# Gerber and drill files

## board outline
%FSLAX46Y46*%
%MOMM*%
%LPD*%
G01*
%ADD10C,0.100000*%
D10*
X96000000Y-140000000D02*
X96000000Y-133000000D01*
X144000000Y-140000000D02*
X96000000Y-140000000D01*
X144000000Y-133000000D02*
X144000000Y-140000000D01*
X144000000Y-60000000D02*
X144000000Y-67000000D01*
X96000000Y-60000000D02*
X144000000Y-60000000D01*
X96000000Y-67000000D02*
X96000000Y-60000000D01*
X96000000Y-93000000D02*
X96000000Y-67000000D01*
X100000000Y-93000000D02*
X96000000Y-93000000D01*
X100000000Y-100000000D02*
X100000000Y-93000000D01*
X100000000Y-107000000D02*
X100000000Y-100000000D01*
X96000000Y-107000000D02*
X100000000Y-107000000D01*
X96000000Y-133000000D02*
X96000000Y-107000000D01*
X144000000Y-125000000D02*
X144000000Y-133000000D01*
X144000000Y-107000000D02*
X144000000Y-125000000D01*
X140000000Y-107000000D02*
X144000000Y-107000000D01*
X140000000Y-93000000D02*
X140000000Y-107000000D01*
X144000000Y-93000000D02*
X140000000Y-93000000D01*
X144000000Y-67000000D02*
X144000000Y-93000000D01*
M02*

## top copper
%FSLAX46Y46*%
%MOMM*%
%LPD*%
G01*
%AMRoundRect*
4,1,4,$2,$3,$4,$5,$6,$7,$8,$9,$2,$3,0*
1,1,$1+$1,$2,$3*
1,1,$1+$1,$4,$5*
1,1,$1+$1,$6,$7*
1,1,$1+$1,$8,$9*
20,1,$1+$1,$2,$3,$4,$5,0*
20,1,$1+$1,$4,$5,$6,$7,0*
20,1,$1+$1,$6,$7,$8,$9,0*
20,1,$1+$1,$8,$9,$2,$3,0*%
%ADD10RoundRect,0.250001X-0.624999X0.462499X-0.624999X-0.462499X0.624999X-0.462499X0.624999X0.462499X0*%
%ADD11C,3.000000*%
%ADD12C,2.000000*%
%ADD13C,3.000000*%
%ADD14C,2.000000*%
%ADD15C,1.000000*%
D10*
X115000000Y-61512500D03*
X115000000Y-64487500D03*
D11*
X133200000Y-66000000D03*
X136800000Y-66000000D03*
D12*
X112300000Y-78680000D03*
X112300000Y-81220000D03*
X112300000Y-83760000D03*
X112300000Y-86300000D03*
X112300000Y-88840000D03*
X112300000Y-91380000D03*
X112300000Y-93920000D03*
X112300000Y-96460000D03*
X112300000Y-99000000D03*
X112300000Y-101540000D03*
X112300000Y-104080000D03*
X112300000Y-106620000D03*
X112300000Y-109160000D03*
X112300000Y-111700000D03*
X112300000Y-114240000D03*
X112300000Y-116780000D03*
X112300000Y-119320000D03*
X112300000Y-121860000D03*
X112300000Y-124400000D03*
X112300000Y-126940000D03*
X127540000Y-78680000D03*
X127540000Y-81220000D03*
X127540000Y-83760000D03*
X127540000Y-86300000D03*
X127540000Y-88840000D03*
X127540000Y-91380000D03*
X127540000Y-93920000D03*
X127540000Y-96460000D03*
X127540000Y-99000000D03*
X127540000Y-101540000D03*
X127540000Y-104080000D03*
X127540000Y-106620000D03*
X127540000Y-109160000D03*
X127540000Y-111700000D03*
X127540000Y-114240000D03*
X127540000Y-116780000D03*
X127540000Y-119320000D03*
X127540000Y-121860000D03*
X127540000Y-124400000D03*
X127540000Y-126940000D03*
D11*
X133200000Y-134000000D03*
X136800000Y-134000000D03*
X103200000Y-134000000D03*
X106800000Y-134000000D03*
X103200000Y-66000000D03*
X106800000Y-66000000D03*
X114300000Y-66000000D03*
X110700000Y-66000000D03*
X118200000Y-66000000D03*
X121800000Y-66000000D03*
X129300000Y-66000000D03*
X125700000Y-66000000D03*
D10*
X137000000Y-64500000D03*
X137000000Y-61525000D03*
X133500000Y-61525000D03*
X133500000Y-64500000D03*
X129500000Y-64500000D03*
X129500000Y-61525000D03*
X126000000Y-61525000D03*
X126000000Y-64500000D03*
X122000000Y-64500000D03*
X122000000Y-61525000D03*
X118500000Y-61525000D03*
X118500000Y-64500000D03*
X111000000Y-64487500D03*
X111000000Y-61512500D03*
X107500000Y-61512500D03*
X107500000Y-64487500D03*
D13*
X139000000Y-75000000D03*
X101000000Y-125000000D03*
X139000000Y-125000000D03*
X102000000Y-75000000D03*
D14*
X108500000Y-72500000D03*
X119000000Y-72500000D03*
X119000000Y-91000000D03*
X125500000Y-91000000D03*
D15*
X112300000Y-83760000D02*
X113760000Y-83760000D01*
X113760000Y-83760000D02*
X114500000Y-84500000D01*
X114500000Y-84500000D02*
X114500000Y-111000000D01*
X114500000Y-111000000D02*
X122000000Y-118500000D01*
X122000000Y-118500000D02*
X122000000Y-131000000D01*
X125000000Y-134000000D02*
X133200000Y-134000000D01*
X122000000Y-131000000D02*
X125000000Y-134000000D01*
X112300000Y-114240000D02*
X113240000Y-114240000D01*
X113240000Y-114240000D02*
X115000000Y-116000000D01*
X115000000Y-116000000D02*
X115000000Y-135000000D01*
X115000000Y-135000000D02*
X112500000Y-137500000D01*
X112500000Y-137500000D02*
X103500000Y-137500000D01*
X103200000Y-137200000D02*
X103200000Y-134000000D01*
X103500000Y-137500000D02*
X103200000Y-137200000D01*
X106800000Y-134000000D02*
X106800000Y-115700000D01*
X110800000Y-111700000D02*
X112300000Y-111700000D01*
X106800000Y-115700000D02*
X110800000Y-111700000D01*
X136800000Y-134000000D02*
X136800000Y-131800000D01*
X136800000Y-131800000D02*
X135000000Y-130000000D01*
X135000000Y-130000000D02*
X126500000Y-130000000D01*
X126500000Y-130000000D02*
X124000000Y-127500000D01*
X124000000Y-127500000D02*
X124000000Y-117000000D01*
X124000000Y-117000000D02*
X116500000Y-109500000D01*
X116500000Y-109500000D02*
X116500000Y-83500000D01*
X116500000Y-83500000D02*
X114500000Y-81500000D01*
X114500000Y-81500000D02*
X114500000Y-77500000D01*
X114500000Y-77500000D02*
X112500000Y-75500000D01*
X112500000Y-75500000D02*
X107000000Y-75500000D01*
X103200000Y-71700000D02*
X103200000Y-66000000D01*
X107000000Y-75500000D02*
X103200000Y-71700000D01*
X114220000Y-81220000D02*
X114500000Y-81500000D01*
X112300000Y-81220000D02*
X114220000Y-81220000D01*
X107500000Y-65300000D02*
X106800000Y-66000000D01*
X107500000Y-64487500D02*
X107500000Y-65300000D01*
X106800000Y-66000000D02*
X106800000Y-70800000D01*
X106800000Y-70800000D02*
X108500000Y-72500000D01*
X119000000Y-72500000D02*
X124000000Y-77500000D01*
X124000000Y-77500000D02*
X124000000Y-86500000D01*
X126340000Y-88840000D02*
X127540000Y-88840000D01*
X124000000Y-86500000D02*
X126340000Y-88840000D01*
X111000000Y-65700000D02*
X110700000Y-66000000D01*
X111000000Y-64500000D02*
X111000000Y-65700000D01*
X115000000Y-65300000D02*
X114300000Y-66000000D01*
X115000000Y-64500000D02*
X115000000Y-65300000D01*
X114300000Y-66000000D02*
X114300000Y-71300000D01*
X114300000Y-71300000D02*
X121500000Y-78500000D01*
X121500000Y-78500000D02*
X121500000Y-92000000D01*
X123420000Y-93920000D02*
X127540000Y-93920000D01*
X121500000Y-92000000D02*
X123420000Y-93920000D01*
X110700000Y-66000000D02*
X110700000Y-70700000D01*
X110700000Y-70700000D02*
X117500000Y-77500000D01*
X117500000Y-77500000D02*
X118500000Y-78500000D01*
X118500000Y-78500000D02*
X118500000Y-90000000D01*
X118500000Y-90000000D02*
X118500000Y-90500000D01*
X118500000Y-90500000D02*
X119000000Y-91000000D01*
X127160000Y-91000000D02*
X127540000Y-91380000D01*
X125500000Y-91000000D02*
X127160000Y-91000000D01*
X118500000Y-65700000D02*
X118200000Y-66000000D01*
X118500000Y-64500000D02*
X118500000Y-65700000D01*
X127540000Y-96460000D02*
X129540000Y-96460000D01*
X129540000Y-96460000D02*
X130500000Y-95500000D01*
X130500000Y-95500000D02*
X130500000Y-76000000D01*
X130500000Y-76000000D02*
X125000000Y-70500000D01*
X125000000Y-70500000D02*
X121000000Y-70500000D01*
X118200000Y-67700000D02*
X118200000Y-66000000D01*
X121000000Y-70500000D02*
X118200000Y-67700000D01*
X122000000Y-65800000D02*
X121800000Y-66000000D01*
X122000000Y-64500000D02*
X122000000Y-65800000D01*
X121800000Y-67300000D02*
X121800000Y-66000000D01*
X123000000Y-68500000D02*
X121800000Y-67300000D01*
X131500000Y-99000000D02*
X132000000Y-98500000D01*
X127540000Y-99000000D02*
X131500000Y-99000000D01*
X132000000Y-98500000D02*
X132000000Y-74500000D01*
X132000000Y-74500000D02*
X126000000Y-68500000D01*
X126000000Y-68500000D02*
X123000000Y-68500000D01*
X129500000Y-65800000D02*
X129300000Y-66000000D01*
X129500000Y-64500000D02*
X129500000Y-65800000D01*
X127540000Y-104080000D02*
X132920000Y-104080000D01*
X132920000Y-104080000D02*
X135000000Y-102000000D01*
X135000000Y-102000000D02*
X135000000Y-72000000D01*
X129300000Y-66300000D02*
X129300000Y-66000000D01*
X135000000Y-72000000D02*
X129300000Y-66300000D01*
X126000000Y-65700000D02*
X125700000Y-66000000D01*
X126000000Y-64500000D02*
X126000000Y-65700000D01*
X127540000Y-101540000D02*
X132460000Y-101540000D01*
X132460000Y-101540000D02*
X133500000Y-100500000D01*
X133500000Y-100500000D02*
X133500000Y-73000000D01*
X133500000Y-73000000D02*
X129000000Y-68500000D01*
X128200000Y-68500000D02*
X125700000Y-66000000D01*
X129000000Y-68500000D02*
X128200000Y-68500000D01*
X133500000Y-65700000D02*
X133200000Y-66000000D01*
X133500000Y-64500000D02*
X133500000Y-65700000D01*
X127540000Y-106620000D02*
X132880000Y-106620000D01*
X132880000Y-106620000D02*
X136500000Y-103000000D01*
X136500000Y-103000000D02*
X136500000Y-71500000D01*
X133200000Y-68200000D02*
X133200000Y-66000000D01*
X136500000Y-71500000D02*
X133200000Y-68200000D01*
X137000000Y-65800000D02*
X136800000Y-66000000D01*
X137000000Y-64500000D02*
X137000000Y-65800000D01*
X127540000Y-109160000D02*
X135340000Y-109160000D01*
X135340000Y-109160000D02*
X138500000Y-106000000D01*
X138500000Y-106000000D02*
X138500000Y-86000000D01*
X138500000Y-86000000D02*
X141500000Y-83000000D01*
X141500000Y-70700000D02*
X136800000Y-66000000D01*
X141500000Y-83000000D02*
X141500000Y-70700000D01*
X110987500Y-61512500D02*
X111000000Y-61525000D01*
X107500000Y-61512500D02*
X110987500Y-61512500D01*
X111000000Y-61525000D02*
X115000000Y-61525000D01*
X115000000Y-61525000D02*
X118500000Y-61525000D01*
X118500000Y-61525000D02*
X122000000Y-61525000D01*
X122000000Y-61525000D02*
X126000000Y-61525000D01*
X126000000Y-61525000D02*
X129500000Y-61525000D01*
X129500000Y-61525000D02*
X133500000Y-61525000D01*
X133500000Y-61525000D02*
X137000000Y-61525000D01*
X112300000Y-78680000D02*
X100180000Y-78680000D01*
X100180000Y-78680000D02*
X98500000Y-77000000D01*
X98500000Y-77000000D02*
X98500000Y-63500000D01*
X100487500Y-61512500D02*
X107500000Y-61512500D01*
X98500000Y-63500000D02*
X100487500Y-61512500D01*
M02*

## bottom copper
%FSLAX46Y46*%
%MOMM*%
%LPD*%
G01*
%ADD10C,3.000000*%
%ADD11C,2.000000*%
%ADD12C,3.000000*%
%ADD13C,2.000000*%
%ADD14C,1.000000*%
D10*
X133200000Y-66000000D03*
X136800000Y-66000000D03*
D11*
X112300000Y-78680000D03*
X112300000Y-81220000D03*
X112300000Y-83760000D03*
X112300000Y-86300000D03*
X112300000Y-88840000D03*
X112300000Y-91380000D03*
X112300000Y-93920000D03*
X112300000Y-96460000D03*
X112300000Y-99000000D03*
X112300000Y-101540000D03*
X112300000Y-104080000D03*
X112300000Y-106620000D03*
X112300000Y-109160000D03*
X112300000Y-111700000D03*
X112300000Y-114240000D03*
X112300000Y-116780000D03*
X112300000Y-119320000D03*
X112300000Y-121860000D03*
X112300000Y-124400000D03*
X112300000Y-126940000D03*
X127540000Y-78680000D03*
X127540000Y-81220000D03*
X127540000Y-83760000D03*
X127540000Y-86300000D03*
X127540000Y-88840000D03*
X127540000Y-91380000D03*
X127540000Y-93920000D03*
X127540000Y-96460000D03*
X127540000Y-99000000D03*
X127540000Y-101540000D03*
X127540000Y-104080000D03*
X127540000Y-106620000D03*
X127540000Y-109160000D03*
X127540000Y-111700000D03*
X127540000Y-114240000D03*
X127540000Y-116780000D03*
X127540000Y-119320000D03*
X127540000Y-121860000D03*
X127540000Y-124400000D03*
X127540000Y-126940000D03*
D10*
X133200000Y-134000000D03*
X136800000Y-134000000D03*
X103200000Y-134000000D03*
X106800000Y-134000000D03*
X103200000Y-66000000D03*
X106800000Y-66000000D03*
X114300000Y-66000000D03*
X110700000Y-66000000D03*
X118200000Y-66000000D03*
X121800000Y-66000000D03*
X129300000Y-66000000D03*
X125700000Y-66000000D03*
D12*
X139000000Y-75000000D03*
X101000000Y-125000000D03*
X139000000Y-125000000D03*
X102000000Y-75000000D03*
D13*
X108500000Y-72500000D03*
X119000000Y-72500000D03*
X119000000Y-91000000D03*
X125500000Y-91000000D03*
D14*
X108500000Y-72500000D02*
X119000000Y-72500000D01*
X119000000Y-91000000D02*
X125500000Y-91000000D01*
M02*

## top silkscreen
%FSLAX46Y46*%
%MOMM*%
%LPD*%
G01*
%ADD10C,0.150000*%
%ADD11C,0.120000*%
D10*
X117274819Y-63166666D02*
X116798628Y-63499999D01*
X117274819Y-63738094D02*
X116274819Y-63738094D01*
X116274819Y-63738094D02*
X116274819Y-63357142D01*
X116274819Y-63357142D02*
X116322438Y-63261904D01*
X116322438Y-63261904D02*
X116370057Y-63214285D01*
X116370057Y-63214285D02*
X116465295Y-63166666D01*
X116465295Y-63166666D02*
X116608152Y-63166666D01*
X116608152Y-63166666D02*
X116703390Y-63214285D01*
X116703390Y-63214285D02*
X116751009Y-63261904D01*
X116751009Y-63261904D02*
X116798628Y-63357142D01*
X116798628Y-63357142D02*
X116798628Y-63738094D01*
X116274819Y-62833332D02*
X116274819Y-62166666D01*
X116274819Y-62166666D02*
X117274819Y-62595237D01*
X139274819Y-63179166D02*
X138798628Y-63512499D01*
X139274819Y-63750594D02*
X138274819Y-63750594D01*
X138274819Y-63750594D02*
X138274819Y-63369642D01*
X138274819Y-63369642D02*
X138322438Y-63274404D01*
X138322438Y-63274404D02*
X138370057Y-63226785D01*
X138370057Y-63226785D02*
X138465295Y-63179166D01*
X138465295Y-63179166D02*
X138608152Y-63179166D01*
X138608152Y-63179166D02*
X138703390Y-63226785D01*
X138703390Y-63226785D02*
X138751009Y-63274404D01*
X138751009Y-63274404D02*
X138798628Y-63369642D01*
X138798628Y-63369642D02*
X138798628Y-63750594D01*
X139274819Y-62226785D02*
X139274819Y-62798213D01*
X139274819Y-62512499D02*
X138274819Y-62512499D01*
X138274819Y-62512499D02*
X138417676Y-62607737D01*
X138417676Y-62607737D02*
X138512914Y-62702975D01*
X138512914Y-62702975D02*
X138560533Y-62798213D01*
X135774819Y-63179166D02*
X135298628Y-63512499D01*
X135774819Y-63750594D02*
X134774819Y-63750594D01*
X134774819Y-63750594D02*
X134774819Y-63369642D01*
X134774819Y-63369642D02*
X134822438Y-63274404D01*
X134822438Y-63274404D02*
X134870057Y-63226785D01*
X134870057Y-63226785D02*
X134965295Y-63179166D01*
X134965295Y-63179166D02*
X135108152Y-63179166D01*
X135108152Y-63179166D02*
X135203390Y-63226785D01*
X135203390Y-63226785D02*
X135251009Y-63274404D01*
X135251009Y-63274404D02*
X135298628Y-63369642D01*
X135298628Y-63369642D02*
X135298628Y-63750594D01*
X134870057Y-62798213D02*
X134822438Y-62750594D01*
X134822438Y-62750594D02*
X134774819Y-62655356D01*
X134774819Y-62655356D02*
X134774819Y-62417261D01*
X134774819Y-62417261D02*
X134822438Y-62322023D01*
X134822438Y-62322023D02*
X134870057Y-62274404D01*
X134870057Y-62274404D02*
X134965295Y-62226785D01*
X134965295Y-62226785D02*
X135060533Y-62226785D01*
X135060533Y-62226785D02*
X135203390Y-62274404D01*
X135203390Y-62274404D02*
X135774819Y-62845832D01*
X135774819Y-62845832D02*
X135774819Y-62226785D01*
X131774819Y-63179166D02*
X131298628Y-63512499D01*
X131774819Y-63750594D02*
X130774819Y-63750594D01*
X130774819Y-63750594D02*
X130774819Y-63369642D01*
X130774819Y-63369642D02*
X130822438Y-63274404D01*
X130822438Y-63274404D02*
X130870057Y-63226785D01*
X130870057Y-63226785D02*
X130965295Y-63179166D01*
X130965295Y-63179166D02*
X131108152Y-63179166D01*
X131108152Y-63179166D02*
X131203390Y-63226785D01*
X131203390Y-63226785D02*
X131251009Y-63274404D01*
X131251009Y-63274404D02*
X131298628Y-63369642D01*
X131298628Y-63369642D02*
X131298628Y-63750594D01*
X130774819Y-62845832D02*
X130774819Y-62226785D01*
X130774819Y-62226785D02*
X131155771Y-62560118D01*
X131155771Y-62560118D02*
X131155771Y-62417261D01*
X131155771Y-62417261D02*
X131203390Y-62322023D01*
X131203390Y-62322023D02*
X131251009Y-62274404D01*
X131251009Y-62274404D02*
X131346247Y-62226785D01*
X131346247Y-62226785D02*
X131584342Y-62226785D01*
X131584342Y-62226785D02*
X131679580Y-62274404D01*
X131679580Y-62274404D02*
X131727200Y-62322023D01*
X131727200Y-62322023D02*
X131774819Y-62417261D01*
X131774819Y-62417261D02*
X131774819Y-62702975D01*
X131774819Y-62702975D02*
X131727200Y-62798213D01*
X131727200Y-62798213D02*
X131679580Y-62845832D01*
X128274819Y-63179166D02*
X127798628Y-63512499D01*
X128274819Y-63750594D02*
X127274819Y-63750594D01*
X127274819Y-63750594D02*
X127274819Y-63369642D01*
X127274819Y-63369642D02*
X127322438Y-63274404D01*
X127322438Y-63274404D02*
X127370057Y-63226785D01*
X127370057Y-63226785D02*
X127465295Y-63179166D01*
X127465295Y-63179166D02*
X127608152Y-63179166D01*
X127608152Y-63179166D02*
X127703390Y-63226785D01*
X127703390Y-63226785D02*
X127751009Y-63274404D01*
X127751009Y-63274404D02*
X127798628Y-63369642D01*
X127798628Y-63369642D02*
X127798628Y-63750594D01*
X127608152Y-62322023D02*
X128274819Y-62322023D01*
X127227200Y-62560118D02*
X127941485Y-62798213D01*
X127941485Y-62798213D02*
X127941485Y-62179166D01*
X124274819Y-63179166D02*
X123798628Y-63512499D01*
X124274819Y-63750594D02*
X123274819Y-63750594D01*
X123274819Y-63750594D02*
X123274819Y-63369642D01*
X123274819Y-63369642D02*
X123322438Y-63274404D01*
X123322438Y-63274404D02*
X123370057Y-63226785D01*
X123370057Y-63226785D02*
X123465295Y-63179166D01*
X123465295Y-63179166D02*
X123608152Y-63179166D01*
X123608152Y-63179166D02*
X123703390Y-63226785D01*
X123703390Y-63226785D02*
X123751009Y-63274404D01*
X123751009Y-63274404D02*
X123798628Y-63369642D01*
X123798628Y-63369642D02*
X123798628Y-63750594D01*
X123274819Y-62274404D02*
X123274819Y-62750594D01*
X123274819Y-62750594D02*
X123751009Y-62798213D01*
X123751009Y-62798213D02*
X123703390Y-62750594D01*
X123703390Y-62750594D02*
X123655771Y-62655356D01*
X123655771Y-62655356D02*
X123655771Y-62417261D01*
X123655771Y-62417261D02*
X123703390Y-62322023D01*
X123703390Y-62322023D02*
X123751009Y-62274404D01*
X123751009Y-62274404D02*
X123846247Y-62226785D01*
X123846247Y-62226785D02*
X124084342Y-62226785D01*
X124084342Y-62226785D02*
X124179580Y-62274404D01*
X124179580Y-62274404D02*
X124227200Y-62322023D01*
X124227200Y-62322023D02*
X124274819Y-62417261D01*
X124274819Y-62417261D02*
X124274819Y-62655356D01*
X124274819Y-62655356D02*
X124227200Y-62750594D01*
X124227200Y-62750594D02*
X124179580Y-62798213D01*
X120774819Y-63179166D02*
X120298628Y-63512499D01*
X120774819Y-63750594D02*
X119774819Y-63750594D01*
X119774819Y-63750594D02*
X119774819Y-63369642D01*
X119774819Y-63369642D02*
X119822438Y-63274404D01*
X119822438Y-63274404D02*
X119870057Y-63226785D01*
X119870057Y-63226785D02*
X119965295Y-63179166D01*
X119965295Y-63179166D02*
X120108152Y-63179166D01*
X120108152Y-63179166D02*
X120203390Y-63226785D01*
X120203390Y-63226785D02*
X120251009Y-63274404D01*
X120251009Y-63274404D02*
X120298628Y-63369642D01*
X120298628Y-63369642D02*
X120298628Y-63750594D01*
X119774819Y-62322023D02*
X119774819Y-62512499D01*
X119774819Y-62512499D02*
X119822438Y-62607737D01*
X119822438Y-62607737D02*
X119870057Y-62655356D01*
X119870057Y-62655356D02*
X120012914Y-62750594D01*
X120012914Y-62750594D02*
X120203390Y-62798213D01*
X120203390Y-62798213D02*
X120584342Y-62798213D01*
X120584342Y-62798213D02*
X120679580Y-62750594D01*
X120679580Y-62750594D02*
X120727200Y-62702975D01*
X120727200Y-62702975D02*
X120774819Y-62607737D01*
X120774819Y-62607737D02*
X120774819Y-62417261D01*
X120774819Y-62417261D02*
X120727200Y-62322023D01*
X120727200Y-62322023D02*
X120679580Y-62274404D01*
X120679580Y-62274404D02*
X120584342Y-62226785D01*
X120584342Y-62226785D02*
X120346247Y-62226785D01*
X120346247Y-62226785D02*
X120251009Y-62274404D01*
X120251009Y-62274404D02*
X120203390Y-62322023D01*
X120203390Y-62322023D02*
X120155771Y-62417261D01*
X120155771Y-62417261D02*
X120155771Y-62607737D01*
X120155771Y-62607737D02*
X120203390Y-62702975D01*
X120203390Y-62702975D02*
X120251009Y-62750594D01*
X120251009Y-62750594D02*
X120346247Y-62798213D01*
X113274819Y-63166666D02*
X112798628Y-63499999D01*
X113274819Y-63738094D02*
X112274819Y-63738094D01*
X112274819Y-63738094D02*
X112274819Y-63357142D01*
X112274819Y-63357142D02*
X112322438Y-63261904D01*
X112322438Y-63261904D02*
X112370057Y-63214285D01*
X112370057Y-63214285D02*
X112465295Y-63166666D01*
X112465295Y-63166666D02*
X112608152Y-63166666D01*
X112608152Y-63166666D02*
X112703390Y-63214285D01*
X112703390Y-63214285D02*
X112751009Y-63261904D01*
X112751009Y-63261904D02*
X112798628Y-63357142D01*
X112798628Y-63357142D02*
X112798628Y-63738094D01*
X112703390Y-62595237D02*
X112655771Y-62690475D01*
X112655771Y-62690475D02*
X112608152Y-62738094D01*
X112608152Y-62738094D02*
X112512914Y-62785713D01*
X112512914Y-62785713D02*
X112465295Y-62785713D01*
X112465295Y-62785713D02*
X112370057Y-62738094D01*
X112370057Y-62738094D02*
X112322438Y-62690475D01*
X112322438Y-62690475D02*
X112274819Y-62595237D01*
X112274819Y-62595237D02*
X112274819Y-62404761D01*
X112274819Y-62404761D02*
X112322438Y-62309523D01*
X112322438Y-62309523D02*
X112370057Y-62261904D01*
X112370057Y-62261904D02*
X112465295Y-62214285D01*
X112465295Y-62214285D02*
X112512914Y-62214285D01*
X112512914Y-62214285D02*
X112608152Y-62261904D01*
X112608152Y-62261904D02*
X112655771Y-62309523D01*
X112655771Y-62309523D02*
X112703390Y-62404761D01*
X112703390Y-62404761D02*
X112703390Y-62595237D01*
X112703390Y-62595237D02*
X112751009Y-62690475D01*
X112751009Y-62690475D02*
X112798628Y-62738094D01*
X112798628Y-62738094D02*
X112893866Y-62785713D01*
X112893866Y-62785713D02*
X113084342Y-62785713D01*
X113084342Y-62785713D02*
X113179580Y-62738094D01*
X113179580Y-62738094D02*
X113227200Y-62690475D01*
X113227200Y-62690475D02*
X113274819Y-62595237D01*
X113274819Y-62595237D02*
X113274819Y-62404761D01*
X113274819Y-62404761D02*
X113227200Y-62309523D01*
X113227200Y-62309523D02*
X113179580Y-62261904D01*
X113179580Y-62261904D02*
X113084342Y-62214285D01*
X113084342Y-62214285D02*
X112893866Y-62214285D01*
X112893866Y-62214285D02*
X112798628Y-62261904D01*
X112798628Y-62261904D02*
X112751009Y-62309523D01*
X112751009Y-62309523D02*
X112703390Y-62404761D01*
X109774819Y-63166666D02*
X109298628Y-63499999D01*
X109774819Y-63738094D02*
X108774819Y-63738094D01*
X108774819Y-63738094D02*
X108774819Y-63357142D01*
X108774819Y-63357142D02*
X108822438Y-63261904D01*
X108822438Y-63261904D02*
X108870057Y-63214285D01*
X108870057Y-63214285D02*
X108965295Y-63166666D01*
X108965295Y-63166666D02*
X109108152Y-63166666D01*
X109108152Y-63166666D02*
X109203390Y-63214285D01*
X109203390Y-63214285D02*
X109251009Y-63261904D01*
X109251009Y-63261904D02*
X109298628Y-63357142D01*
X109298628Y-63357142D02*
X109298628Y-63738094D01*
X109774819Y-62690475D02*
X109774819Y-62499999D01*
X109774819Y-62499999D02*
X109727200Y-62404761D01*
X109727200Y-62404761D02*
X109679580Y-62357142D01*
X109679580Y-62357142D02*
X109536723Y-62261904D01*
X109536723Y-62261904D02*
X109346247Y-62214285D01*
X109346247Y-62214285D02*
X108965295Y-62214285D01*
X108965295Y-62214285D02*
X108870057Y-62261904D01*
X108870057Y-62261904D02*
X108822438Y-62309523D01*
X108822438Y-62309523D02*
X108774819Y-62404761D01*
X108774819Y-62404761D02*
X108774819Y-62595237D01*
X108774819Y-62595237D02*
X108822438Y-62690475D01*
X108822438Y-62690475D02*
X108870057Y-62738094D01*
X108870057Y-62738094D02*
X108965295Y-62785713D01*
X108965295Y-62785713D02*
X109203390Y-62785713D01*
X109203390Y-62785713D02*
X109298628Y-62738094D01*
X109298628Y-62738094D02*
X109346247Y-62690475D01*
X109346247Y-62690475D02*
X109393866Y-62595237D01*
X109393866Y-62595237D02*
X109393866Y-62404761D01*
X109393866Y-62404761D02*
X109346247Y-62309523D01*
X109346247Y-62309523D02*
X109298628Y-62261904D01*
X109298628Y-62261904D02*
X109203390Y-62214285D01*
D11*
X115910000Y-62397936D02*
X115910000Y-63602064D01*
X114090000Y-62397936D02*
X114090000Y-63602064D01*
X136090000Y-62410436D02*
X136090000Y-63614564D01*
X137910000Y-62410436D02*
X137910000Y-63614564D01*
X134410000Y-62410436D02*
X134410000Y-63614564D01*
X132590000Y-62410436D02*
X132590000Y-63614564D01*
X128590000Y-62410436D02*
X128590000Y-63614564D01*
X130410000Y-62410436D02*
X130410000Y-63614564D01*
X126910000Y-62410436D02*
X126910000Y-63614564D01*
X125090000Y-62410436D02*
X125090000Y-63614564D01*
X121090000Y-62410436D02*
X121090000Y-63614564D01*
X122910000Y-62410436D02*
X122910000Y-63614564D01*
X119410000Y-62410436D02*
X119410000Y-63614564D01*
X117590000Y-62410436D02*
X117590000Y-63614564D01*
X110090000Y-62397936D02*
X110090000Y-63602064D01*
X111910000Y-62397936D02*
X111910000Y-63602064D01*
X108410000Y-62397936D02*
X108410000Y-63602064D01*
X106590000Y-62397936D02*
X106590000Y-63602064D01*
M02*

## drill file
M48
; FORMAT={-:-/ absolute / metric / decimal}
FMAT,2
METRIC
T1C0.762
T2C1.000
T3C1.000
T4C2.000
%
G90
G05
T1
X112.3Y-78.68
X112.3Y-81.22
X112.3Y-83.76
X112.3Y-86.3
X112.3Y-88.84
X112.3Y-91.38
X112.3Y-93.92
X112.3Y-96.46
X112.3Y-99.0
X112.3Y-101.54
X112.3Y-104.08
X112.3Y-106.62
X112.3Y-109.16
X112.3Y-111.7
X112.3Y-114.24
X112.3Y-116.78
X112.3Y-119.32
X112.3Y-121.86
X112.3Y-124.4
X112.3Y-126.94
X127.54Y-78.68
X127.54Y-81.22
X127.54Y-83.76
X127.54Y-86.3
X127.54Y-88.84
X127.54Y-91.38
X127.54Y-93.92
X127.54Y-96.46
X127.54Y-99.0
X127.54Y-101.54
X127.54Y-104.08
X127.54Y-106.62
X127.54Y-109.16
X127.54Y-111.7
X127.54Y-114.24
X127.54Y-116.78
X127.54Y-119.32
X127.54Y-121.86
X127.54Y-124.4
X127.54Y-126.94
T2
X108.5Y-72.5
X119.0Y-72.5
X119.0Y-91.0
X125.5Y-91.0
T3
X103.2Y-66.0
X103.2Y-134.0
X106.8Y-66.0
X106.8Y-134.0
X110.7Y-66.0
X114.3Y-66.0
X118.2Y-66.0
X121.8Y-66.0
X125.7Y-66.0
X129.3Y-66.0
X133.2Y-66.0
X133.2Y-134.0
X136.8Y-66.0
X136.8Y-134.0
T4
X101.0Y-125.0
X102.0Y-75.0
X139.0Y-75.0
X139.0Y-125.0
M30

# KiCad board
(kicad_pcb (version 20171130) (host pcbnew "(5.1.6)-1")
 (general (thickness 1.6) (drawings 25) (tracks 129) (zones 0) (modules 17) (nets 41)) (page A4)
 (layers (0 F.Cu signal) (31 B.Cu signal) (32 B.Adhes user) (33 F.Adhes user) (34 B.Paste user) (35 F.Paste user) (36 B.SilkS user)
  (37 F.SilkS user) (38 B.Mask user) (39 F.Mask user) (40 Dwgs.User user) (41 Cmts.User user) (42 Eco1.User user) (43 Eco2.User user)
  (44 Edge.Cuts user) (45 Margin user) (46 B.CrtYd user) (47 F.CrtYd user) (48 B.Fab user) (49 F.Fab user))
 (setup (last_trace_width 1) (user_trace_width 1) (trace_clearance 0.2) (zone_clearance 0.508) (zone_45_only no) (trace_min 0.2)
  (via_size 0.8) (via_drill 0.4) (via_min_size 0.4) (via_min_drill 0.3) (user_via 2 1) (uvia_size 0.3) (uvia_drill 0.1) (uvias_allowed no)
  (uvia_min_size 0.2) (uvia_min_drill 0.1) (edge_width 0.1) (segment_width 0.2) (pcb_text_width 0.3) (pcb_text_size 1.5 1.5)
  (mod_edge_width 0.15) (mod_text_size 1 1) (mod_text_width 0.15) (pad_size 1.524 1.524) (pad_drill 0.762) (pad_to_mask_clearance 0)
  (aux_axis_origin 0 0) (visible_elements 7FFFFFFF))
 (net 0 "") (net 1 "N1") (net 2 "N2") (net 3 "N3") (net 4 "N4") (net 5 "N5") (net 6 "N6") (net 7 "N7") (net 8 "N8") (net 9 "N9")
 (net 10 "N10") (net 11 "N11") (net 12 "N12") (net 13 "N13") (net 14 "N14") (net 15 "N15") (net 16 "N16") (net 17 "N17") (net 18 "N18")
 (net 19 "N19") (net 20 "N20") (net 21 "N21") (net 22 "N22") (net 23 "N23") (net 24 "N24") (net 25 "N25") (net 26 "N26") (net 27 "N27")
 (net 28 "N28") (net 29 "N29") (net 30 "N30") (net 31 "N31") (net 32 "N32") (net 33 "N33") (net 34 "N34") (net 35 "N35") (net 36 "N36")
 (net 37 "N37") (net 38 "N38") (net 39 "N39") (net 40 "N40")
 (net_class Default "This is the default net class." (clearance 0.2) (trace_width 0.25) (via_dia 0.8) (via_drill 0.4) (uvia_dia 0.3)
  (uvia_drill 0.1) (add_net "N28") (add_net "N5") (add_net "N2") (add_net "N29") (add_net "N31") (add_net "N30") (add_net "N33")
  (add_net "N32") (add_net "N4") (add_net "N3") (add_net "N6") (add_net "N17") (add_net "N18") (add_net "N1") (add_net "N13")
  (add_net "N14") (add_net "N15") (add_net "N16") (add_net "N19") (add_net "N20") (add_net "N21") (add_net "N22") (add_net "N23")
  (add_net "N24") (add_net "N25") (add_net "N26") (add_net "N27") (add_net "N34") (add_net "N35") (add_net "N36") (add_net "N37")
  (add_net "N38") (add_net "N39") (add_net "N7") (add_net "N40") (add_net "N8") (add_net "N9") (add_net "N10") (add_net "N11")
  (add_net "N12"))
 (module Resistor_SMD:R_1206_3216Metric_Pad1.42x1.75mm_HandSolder (layer F.Cu) (at 115 63 270)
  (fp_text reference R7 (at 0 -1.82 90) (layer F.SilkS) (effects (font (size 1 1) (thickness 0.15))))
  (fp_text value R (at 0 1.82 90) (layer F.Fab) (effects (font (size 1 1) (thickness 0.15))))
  (fp_line (start -0.602064 -0.91) (end 0.602064 -0.91) (layer F.SilkS) (width 0.12))
  (fp_line (start -0.602064 0.91) (end 0.602064 0.91) (layer F.SilkS) (width 0.12))
  (pad 1 smd roundrect (at -1.4875 0 270) (size 1.425 1.75) (layers F.Cu F.Paste F.Mask) (roundrect_rratio 0.175439) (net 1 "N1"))
  (pad 2 smd roundrect (at 1.4875 0 270) (size 1.425 1.75) (layers F.Cu F.Paste F.Mask) (roundrect_rratio 0.175439) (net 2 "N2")))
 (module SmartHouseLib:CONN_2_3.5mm (layer B.Cu) (at 135 66 180)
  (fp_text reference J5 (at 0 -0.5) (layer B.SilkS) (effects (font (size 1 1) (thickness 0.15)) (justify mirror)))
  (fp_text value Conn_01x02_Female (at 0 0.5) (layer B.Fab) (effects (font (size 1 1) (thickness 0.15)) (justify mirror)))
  (pad 2 thru_hole circle (at 1.8 0 180) (size 3 3) (drill 1) (layers *.Cu *.Mask) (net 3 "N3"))
  (pad 1 thru_hole circle (at -1.8 0 180) (size 3 3) (drill 1) (layers *.Cu *.Mask) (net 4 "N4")))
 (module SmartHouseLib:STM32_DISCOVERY (layer B.Cu) (at 125 99 180)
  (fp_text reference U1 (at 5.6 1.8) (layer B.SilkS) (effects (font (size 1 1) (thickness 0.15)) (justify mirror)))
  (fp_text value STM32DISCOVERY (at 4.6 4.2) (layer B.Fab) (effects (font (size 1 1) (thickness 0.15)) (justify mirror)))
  (pad 1 thru_hole circle (at 12.7 20.32 180) (size 2 2) (drill 0.762) (layers *.Cu *.Mask) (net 1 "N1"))
  (pad 2 thru_hole circle (at 12.7 17.78 180) (size 2 2) (drill 0.762) (layers *.Cu *.Mask) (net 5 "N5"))
  (pad 3 thru_hole circle (at 12.7 15.24 180) (size 2 2) (drill 0.762) (layers *.Cu *.Mask) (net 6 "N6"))
  (pad 4 thru_hole circle (at 12.7 12.7 180) (size 2 2) (drill 0.762) (layers *.Cu *.Mask) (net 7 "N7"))
  (pad 5 thru_hole circle (at 12.7 10.16 180) (size 2 2) (drill 0.762) (layers *.Cu *.Mask) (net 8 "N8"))
  (pad 6 thru_hole circle (at 12.7 7.62 180) (size 2 2) (drill 0.762) (layers *.Cu *.Mask) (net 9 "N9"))
  (pad 7 thru_hole circle (at 12.7 5.08 180) (size 2 2) (drill 0.762) (layers *.Cu *.Mask) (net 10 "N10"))
  (pad 8 thru_hole circle (at 12.7 2.54 180) (size 2 2) (drill 0.762) (layers *.Cu *.Mask) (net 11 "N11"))
  (pad 9 thru_hole circle (at 12.7 0 180) (size 2 2) (drill 0.762) (layers *.Cu *.Mask) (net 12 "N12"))
  (pad 10 thru_hole circle (at 12.7 -2.54 180) (size 2 2) (drill 0.762) (layers *.Cu *.Mask) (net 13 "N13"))
  (pad 11 thru_hole circle (at 12.7 -5.08 180) (size 2 2) (drill 0.762) (layers *.Cu *.Mask) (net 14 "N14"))
  (pad 12 thru_hole circle (at 12.7 -7.62 180) (size 2 2) (drill 0.762) (layers *.Cu *.Mask) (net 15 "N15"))
  (pad 13 thru_hole circle (at 12.7 -10.16 180) (size 2 2) (drill 0.762) (layers *.Cu *.Mask) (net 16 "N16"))
  (pad 14 thru_hole circle (at 12.7 -12.7 180) (size 2 2) (drill 0.762) (layers *.Cu *.Mask) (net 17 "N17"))
  (pad 15 thru_hole circle (at 12.7 -15.24 180) (size 2 2) (drill 0.762) (layers *.Cu *.Mask) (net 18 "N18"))
  (pad 16 thru_hole circle (at 12.7 -17.78 180) (size 2 2) (drill 0.762) (layers *.Cu *.Mask) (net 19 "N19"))
  (pad 17 thru_hole circle (at 12.7 -20.32 180) (size 2 2) (drill 0.762) (layers *.Cu *.Mask) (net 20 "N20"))
  (pad 18 thru_hole circle (at 12.7 -22.86 180) (size 2 2) (drill 0.762) (layers *.Cu *.Mask) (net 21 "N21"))
  (pad 19 thru_hole circle (at 12.7 -25.4 180) (size 2 2) (drill 0.762) (layers *.Cu *.Mask) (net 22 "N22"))
  (pad 20 thru_hole circle (at 12.7 -27.94 180) (size 2 2) (drill 0.762) (layers *.Cu *.Mask) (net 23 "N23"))
  (pad 21 thru_hole circle (at -2.54 20.32 180) (size 2 2) (drill 0.762) (layers *.Cu *.Mask) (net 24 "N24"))
  (pad 22 thru_hole circle (at -2.54 17.78 180) (size 2 2) (drill 0.762) (layers *.Cu *.Mask) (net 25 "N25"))
  (pad 23 thru_hole circle (at -2.54 15.24 180) (size 2 2) (drill 0.762) (layers *.Cu *.Mask) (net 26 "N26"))
  (pad 24 thru_hole circle (at -2.54 12.7 180) (size 2 2) (drill 0.762) (layers *.Cu *.Mask) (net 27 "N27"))
  (pad 25 thru_hole circle (at -2.54 10.16 180) (size 2 2) (drill 0.762) (layers *.Cu *.Mask) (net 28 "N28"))
  (pad 26 thru_hole circle (at -2.54 7.62 180) (size 2 2) (drill 0.762) (layers *.Cu *.Mask) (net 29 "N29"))
  (pad 27 thru_hole circle (at -2.54 5.08 180) (size 2 2) (drill 0.762) (layers *.Cu *.Mask) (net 2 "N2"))
  (pad 28 thru_hole circle (at -2.54 2.54 180) (size 2 2) (drill 0.762) (layers *.Cu *.Mask) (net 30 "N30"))
  (pad 29 thru_hole circle (at -2.54 0 180) (size 2 2) (drill 0.762) (layers *.Cu *.Mask) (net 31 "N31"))
  (pad 30 thru_hole circle (at -2.54 -2.54 180) (size 2 2) (drill 0.762) (layers *.Cu *.Mask) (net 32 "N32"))
  (pad 31 thru_hole circle (at -2.54 -5.08 180) (size 2 2) (drill 0.762) (layers *.Cu *.Mask) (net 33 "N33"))
  (pad 32 thru_hole circle (at -2.54 -7.62 180) (size 2 2) (drill 0.762) (layers *.Cu *.Mask) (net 3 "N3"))
  (pad 33 thru_hole circle (at -2.54 -10.16 180) (size 2 2) (drill 0.762) (layers *.Cu *.Mask) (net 4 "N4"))
  (pad 34 thru_hole circle (at -2.54 -12.7 180) (size 2 2) (drill 0.762) (layers *.Cu *.Mask) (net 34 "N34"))
  (pad 35 thru_hole circle (at -2.54 -15.24 180) (size 2 2) (drill 0.762) (layers *.Cu *.Mask) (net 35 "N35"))
  (pad 36 thru_hole circle (at -2.54 -17.78 180) (size 2 2) (drill 0.762) (layers *.Cu *.Mask) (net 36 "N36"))
  (pad 37 thru_hole circle (at -2.54 -20.32 180) (size 2 2) (drill 0.762) (layers *.Cu *.Mask) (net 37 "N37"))
  (pad 38 thru_hole circle (at -2.54 -22.86 180) (size 2 2) (drill 0.762) (layers *.Cu *.Mask) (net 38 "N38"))
  (pad 39 thru_hole circle (at -2.54 -25.4 180) (size 2 2) (drill 0.762) (layers *.Cu *.Mask) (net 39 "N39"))
  (pad 40 thru_hole circle (at -2.54 -27.94 180) (size 2 2) (drill 0.762) (layers *.Cu *.Mask) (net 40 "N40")))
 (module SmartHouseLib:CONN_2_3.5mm (layer B.Cu) (at 135 134)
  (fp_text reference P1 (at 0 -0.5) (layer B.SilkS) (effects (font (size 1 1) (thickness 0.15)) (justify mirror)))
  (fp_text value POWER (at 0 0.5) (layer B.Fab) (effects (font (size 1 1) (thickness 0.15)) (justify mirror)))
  (pad 1 thru_hole circle (at -1.8 0) (size 3 3) (drill 1) (layers *.Cu *.Mask) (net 6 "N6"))
  (pad 2 thru_hole circle (at 1.8 0) (size 3 3) (drill 1) (layers *.Cu *.Mask) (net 5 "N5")))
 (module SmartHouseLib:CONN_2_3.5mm (layer B.Cu) (at 105 134 180)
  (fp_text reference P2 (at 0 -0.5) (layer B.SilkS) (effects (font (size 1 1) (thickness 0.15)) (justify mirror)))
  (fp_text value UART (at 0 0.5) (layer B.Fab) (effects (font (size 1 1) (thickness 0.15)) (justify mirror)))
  (pad 2 thru_hole circle (at 1.8 0 180) (size 3 3) (drill 1) (layers *.Cu *.Mask) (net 18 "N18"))
  (pad 1 thru_hole circle (at -1.8 0 180) (size 3 3) (drill 1) (layers *.Cu *.Mask) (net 17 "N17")))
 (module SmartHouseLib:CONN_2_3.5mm (layer B.Cu) (at 105 66 180)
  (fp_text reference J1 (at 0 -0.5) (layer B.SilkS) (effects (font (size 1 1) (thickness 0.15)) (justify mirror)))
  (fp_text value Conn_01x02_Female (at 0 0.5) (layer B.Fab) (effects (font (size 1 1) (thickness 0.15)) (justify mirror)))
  (pad 2 thru_hole circle (at 1.8 0 180) (size 3 3) (drill 1) (layers *.Cu *.Mask) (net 5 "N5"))
  (pad 1 thru_hole circle (at -1.8 0 180) (size 3 3) (drill 1) (layers *.Cu *.Mask) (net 28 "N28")))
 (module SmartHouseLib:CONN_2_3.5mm (layer B.Cu) (at 112.5 66 180)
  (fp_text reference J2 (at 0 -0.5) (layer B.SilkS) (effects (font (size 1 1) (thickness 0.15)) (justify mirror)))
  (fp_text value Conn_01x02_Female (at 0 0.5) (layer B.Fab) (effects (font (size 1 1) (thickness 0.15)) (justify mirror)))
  (pad 1 thru_hole circle (at -1.8 0 180) (size 3 3) (drill 1) (layers *.Cu *.Mask) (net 2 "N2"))
  (pad 2 thru_hole circle (at 1.8 0 180) (size 3 3) (drill 1) (layers *.Cu *.Mask) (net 29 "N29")))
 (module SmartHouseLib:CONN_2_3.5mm (layer B.Cu) (at 120 66 180)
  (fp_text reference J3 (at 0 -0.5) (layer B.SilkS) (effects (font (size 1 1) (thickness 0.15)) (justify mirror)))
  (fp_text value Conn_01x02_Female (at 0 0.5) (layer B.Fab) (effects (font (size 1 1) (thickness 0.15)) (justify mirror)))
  (pad 2 thru_hole circle (at 1.8 0 180) (size 3 3) (drill 1) (layers *.Cu *.Mask) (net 30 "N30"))
  (pad 1 thru_hole circle (at -1.8 0 180) (size 3 3) (drill 1) (layers *.Cu *.Mask) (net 31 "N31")))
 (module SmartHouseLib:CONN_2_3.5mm (layer B.Cu) (at 127.5 66 180)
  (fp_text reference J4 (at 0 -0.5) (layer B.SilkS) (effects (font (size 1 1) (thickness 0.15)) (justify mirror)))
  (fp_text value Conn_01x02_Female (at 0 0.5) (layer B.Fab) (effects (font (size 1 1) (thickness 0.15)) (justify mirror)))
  (pad 1 thru_hole circle (at -1.8 0 180) (size 3 3) (drill 1) (layers *.Cu *.Mask) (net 33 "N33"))
  (pad 2 thru_hole circle (at 1.8 0 180) (size 3 3) (drill 1) (layers *.Cu *.Mask) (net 32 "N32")))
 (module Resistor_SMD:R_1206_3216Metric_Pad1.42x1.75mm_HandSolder (layer F.Cu) (at 137 63.0125 270)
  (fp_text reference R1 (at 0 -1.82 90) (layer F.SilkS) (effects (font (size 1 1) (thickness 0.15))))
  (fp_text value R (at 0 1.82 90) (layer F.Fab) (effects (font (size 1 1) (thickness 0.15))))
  (fp_line (start -0.602064 0.91) (end 0.602064 0.91) (layer F.SilkS) (width 0.12))
  (fp_line (start -0.602064 -0.91) (end 0.602064 -0.91) (layer F.SilkS) (width 0.12))
  (pad 2 smd roundrect (at 1.4875 0 270) (size 1.425 1.75) (layers F.Cu F.Paste F.Mask) (roundrect_rratio 0.175439) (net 4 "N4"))
  (pad 1 smd roundrect (at -1.4875 0 270) (size 1.425 1.75) (layers F.Cu F.Paste F.Mask) (roundrect_rratio 0.175439) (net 1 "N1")))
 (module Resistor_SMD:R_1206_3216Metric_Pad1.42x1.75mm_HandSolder (layer F.Cu) (at 133.5 63.0125 270)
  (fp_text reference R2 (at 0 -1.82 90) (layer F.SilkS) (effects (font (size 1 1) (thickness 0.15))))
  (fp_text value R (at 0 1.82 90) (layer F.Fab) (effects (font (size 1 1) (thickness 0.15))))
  (fp_line (start -0.602064 -0.91) (end 0.602064 -0.91) (layer F.SilkS) (width 0.12))
  (fp_line (start -0.602064 0.91) (end 0.602064 0.91) (layer F.SilkS) (width 0.12))
  (pad 1 smd roundrect (at -1.4875 0 270) (size 1.425 1.75) (layers F.Cu F.Paste F.Mask) (roundrect_rratio 0.175439) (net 1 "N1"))
  (pad 2 smd roundrect (at 1.4875 0 270) (size 1.425 1.75) (layers F.Cu F.Paste F.Mask) (roundrect_rratio 0.175439) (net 3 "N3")))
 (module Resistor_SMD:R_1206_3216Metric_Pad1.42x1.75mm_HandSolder (layer F.Cu) (at 129.5 63.0125 270)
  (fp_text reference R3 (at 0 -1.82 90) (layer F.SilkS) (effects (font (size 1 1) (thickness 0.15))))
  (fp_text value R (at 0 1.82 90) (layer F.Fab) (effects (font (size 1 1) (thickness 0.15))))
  (fp_line (start -0.602064 0.91) (end 0.602064 0.91) (layer F.SilkS) (width 0.12))
  (fp_line (start -0.602064 -0.91) (end 0.602064 -0.91) (layer F.SilkS) (width 0.12))
  (pad 2 smd roundrect (at 1.4875 0 270) (size 1.425 1.75) (layers F.Cu F.Paste F.Mask) (roundrect_rratio 0.175439) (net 33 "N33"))
  (pad 1 smd roundrect (at -1.4875 0 270) (size 1.425 1.75) (layers F.Cu F.Paste F.Mask) (roundrect_rratio 0.175439) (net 1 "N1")))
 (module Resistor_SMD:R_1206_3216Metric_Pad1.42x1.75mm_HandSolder (layer F.Cu) (at 126 63.0125 270)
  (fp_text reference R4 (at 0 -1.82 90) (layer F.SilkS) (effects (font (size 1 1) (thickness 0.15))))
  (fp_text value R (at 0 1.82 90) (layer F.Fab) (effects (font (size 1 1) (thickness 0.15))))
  (fp_line (start -0.602064 -0.91) (end 0.602064 -0.91) (layer F.SilkS) (width 0.12))
  (fp_line (start -0.602064 0.91) (end 0.602064 0.91) (layer F.SilkS) (width 0.12))
  (pad 1 smd roundrect (at -1.4875 0 270) (size 1.425 1.75) (layers F.Cu F.Paste F.Mask) (roundrect_rratio 0.175439) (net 1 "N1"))
  (pad 2 smd roundrect (at 1.4875 0 270) (size 1.425 1.75) (layers F.Cu F.Paste F.Mask) (roundrect_rratio 0.175439) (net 32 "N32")))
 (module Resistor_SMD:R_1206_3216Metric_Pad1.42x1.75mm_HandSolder (layer F.Cu) (at 122 63.0125 270)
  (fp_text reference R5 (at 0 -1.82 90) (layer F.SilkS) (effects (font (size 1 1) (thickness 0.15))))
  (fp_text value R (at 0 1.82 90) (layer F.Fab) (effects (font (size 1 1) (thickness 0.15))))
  (fp_line (start -0.602064 0.91) (end 0.602064 0.91) (layer F.SilkS) (width 0.12))
  (fp_line (start -0.602064 -0.91) (end 0.602064 -0.91) (layer F.SilkS) (width 0.12))
  (pad 2 smd roundrect (at 1.4875 0 270) (size 1.425 1.75) (layers F.Cu F.Paste F.Mask) (roundrect_rratio 0.175439) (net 31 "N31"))
  (pad 1 smd roundrect (at -1.4875 0 270) (size 1.425 1.75) (layers F.Cu F.Paste F.Mask) (roundrect_rratio 0.175439) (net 1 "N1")))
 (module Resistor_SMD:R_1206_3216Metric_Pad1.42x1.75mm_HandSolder (layer F.Cu) (at 118.5 63.0125 270)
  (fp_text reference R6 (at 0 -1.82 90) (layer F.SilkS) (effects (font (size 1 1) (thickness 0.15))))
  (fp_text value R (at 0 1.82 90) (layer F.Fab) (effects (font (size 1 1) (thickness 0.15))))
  (fp_line (start -0.602064 -0.91) (end 0.602064 -0.91) (layer F.SilkS) (width 0.12))
  (fp_line (start -0.602064 0.91) (end 0.602064 0.91) (layer F.SilkS) (width 0.12))
  (pad 1 smd roundrect (at -1.4875 0 270) (size 1.425 1.75) (layers F.Cu F.Paste F.Mask) (roundrect_rratio 0.175439) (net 1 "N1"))
  (pad 2 smd roundrect (at 1.4875 0 270) (size 1.425 1.75) (layers F.Cu F.Paste F.Mask) (roundrect_rratio 0.175439) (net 30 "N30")))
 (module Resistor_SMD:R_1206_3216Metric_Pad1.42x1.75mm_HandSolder (layer F.Cu) (at 111 63 270)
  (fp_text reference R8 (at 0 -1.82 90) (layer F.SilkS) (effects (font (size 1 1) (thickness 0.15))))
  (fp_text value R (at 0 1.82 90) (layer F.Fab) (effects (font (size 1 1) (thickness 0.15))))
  (fp_line (start -0.602064 0.91) (end 0.602064 0.91) (layer F.SilkS) (width 0.12))
  (fp_line (start -0.602064 -0.91) (end 0.602064 -0.91) (layer F.SilkS) (width 0.12))
  (pad 2 smd roundrect (at 1.4875 0 270) (size 1.425 1.75) (layers F.Cu F.Paste F.Mask) (roundrect_rratio 0.175439) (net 29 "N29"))
  (pad 1 smd roundrect (at -1.4875 0 270) (size 1.425 1.75) (layers F.Cu F.Paste F.Mask) (roundrect_rratio 0.175439) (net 1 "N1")))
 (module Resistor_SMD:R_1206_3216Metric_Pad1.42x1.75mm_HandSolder (layer F.Cu) (at 107.5 63 270)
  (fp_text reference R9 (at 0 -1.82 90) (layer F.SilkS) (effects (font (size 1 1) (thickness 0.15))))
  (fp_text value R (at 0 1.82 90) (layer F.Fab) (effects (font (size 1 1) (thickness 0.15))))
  (fp_line (start -0.602064 -0.91) (end 0.602064 -0.91) (layer F.SilkS) (width 0.12))
  (fp_line (start -0.602064 0.91) (end 0.602064 0.91) (layer F.SilkS) (width 0.12))
  (pad 1 smd roundrect (at -1.4875 0 270) (size 1.425 1.75) (layers F.Cu F.Paste F.Mask) (roundrect_rratio 0.175439) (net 1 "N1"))
  (pad 2 smd roundrect (at 1.4875 0 270) (size 1.425 1.75) (layers F.Cu F.Paste F.Mask) (roundrect_rratio 0.175439) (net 28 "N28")))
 (gr_line (start 96 140) (end 96 133) (layer Edge.Cuts) (width 0.1))
 (gr_line (start 144 140) (end 96 140) (layer Edge.Cuts) (width 0.1))
 (gr_line (start 144 133) (end 144 140) (layer Edge.Cuts) (width 0.1))
 (gr_line (start 144 60) (end 144 67) (layer Edge.Cuts) (width 0.1))
 (gr_line (start 96 60) (end 144 60) (layer Edge.Cuts) (width 0.1))
 (gr_line (start 96 67) (end 96 60) (layer Edge.Cuts) (width 0.1))
 (gr_line (start 96 93) (end 96 67) (layer Edge.Cuts) (width 0.1))
 (gr_line (start 100 93) (end 96 93) (layer Edge.Cuts) (width 0.1))
 (gr_line (start 100 100) (end 100 93) (layer Edge.Cuts) (width 0.1))
 (gr_line (start 100 107) (end 100 100) (layer Edge.Cuts) (width 0.1))
 (gr_line (start 96 107) (end 100 107) (layer Edge.Cuts) (width 0.1))
 (gr_line (start 96 133) (end 96 107) (layer Edge.Cuts) (width 0.1))
 (gr_line (start 144 125) (end 144 133) (layer Edge.Cuts) (width 0.1))
 (gr_line (start 144 107) (end 144 125) (layer Edge.Cuts) (width 0.1))
 (gr_line (start 140 107) (end 144 107) (layer Edge.Cuts) (width 0.1))
 (gr_line (start 140 93) (end 140 107) (layer Edge.Cuts) (width 0.1))
 (gr_line (start 144 93) (end 140 93) (layer Edge.Cuts) (width 0.1))
 (gr_line (start 144 67) (end 144 93) (layer Edge.Cuts) (width 0.1))
 (via (at 139 75) (size 3) (drill 2) (layers F.Cu B.Cu) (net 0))
 (via (at 101 125) (size 3) (drill 2) (layers F.Cu B.Cu) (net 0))
 (via (at 139 125) (size 3) (drill 2) (layers F.Cu B.Cu) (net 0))
 (via (at 102 75) (size 3) (drill 2) (layers F.Cu B.Cu) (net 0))
 (segment (start 112.3 83.76) (end 113.76 83.76) (width 1) (layer F.Cu) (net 6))
 (segment (start 113.76 83.76) (end 114.5 84.5) (width 1) (layer F.Cu) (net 6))
 (segment (start 114.5 84.5) (end 114.5 111) (width 1) (layer F.Cu) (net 6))
 (segment (start 114.5 111) (end 122 118.5) (width 1) (layer F.Cu) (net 6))
 (segment (start 122 118.5) (end 122 131) (width 1) (layer F.Cu) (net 6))
 (segment (start 125 134) (end 133.2 134) (width 1) (layer F.Cu) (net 6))
 (segment (start 122 131) (end 125 134) (width 1) (layer F.Cu) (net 6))
 (segment (start 112.3 114.24) (end 113.24 114.24) (width 1) (layer F.Cu) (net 18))
 (segment (start 113.24 114.24) (end 115 116) (width 1) (layer F.Cu) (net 18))
 (segment (start 115 116) (end 115 135) (width 1) (layer F.Cu) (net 18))
 (segment (start 115 135) (end 112.5 137.5) (width 1) (layer F.Cu) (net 18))
 (segment (start 112.5 137.5) (end 103.5 137.5) (width 1) (layer F.Cu) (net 18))
 (segment (start 103.2 137.2) (end 103.2 134) (width 1) (layer F.Cu) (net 18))
 (segment (start 103.5 137.5) (end 103.2 137.2) (width 1) (layer F.Cu) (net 18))
 (segment (start 106.8 134) (end 106.8 115.7) (width 1) (layer F.Cu) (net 17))
 (segment (start 110.8 111.7) (end 112.3 111.7) (width 1) (layer F.Cu) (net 17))
 (segment (start 106.8 115.7) (end 110.8 111.7) (width 1) (layer F.Cu) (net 17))
 (segment (start 136.8 134) (end 136.8 131.8) (width 1) (layer F.Cu) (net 5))
 (segment (start 136.8 131.8) (end 135 130) (width 1) (layer F.Cu) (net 5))
 (segment (start 135 130) (end 126.5 130) (width 1) (layer F.Cu) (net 5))
 (segment (start 126.5 130) (end 124 127.5) (width 1) (layer F.Cu) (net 5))
 (segment (start 124 127.5) (end 124 117) (width 1) (layer F.Cu) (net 5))
 (segment (start 124 117) (end 116.5 109.5) (width 1) (layer F.Cu) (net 5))
 (segment (start 116.5 109.5) (end 116.5 83.5) (width 1) (layer F.Cu) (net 5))
 (segment (start 116.5 83.5) (end 114.5 81.5) (width 1) (layer F.Cu) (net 5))
 (segment (start 114.5 81.5) (end 114.5 77.5) (width 1) (layer F.Cu) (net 5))
 (segment (start 114.5 77.5) (end 112.5 75.5) (width 1) (layer F.Cu) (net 5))
 (segment (start 112.5 75.5) (end 107 75.5) (width 1) (layer F.Cu) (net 5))
 (segment (start 103.2 71.7) (end 103.2 66) (width 1) (layer F.Cu) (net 5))
 (segment (start 107 75.5) (end 103.2 71.7) (width 1) (layer F.Cu) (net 5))
 (segment (start 114.22 81.22) (end 114.5 81.5) (width 1) (layer F.Cu) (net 5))
 (segment (start 112.3 81.22) (end 114.22 81.22) (width 1) (layer F.Cu) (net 5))
 (segment (start 107.5 65.3) (end 106.8 66) (width 1) (layer F.Cu) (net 28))
 (segment (start 107.5 64.4875) (end 107.5 65.3) (width 1) (layer F.Cu) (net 28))
 (via (at 108.5 72.5) (size 2) (drill 1) (layers F.Cu B.Cu) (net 28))
 (segment (start 106.8 66) (end 106.8 70.8) (width 1) (layer F.Cu) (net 28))
 (segment (start 106.8 70.8) (end 108.5 72.5) (width 1) (layer F.Cu) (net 28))
 (via (at 119 72.5) (size 2) (drill 1) (layers F.Cu B.Cu) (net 28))
 (segment (start 108.5 72.5) (end 119 72.5) (width 1) (layer B.Cu) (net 28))
 (segment (start 119 72.5) (end 124 77.5) (width 1) (layer F.Cu) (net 28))
 (segment (start 124 77.5) (end 124 86.5) (width 1) (layer F.Cu) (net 28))
 (segment (start 126.34 88.84) (end 127.54 88.84) (width 1) (layer F.Cu) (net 28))
 (segment (start 124 86.5) (end 126.34 88.84) (width 1) (layer F.Cu) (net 28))
 (segment (start 111 65.7) (end 110.7 66) (width 1) (layer F.Cu) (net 29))
 (segment (start 111 64.5) (end 111 65.7) (width 1) (layer F.Cu) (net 29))
 (segment (start 115 65.3) (end 114.3 66) (width 1) (layer F.Cu) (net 2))
 (segment (start 115 64.5) (end 115 65.3) (width 1) (layer F.Cu) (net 2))
 (segment (start 114.3 66) (end 114.3 71.3) (width 1) (layer F.Cu) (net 2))
 (segment (start 114.3 71.3) (end 121.5 78.5) (width 1) (layer F.Cu) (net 2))
 (segment (start 121.5 78.5) (end 121.5 92) (width 1) (layer F.Cu) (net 2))
 (segment (start 123.42 93.92) (end 127.54 93.92) (width 1) (layer F.Cu) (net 2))
 (segment (start 121.5 92) (end 123.42 93.92) (width 1) (layer F.Cu) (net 2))
 (segment (start 110.7 66) (end 110.7 70.7) (width 1) (layer F.Cu) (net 29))
 (segment (start 110.7 70.7) (end 117.5 77.5) (width 1) (layer F.Cu) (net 29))
 (segment (start 117.5 77.5) (end 118.5 78.5) (width 1) (layer F.Cu) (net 29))
 (segment (start 118.5 78.5) (end 118.5 90) (width 1) (layer F.Cu) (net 29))
 (via (at 119 91) (size 2) (drill 1) (layers F.Cu B.Cu) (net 29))
 (segment (start 118.5 90) (end 118.5 90.5) (width 1) (layer F.Cu) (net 29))
 (segment (start 118.5 90.5) (end 119 91) (width 1) (layer F.Cu) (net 29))
 (via (at 125.5 91) (size 2) (drill 1) (layers F.Cu B.Cu) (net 29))
 (segment (start 119 91) (end 125.5 91) (width 1) (layer B.Cu) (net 29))
 (segment (start 127.16 91) (end 127.54 91.38) (width 1) (layer F.Cu) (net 29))
 (segment (start 125.5 91) (end 127.16 91) (width 1) (layer F.Cu) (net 29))
 (segment (start 118.5 65.7) (end 118.2 66) (width 1) (layer F.Cu) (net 30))
 (segment (start 118.5 64.5) (end 118.5 65.7) (width 1) (layer F.Cu) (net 30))
 (segment (start 127.54 96.46) (end 129.54 96.46) (width 1) (layer F.Cu) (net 30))
 (segment (start 129.54 96.46) (end 130.5 95.5) (width 1) (layer F.Cu) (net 30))
 (segment (start 130.5 95.5) (end 130.5 76) (width 1) (layer F.Cu) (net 30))
 (segment (start 130.5 76) (end 125 70.5) (width 1) (layer F.Cu) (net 30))
 (segment (start 125 70.5) (end 121 70.5) (width 1) (layer F.Cu) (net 30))
 (segment (start 118.2 67.7) (end 118.2 66) (width 1) (layer F.Cu) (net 30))
 (segment (start 121 70.5) (end 118.2 67.7) (width 1) (layer F.Cu) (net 30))
 (segment (start 122 65.8) (end 121.8 66) (width 1) (layer F.Cu) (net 31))
 (segment (start 122 64.5) (end 122 65.8) (width 1) (layer F.Cu) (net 31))
 (segment (start 121.8 67.3) (end 121.8 66) (width 1) (layer F.Cu) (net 31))
 (segment (start 123 68.5) (end 121.8 67.3) (width 1) (layer F.Cu) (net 31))
 (segment (start 131.5 99) (end 132 98.5) (width 1) (layer F.Cu) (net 31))
 (segment (start 127.54 99) (end 131.5 99) (width 1) (layer F.Cu) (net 31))
 (segment (start 132 98.5) (end 132 74.5) (width 1) (layer F.Cu) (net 31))
 (segment (start 132 74.5) (end 126 68.5) (width 1) (layer F.Cu) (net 31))
 (segment (start 126 68.5) (end 123 68.5) (width 1) (layer F.Cu) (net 31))
 (segment (start 129.5 65.8) (end 129.3 66) (width 1) (layer F.Cu) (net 33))
 (segment (start 129.5 64.5) (end 129.5 65.8) (width 1) (layer F.Cu) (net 33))
 (segment (start 127.54 104.08) (end 132.92 104.08) (width 1) (layer F.Cu) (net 33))
 (segment (start 132.92 104.08) (end 135 102) (width 1) (layer F.Cu) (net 33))
 (segment (start 135 102) (end 135 72) (width 1) (layer F.Cu) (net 33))
 (segment (start 129.3 66.3) (end 129.3 66) (width 1) (layer F.Cu) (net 33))
 (segment (start 135 72) (end 129.3 66.3) (width 1) (layer F.Cu) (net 33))
 (segment (start 126 65.7) (end 125.7 66) (width 1) (layer F.Cu) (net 32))
 (segment (start 126 64.5) (end 126 65.7) (width 1) (layer F.Cu) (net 32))
 (segment (start 127.54 101.54) (end 132.46 101.54) (width 1) (layer F.Cu) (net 32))
 (segment (start 132.46 101.54) (end 133.5 100.5) (width 1) (layer F.Cu) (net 32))
 (segment (start 133.5 100.5) (end 133.5 73) (width 1) (layer F.Cu) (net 32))
 (segment (start 133.5 73) (end 129 68.5) (width 1) (layer F.Cu) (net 32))
 (segment (start 128.2 68.5) (end 125.7 66) (width 1) (layer F.Cu) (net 32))
 (segment (start 129 68.5) (end 128.2 68.5) (width 1) (layer F.Cu) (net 32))
 (segment (start 133.5 65.7) (end 133.2 66) (width 1) (layer F.Cu) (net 3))
 (segment (start 133.5 64.5) (end 133.5 65.7) (width 1) (layer F.Cu) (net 3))
 (segment (start 127.54 106.62) (end 132.88 106.62) (width 1) (layer F.Cu) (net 3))
 (segment (start 132.88 106.62) (end 136.5 103) (width 1) (layer F.Cu) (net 3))
 (segment (start 136.5 103) (end 136.5 71.5) (width 1) (layer F.Cu) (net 3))
 (segment (start 133.2 68.2) (end 133.2 66) (width 1) (layer F.Cu) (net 3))
 (segment (start 136.5 71.5) (end 133.2 68.2) (width 1) (layer F.Cu) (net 3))
 (segment (start 137 65.8) (end 136.8 66) (width 1) (layer F.Cu) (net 4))
 (segment (start 137 64.5) (end 137 65.8) (width 1) (layer F.Cu) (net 4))
 (segment (start 127.54 109.16) (end 135.34 109.16) (width 1) (layer F.Cu) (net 4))
 (segment (start 135.34 109.16) (end 138.5 106) (width 1) (layer F.Cu) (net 4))
 (segment (start 138.5 106) (end 138.5 86) (width 1) (layer F.Cu) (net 4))
 (segment (start 138.5 86) (end 141.5 83) (width 1) (layer F.Cu) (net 4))
 (segment (start 141.5 70.7) (end 136.8 66) (width 1) (layer F.Cu) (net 4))
 (segment (start 141.5 83) (end 141.5 70.7) (width 1) (layer F.Cu) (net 4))
 (segment (start 110.9875 61.5125) (end 111 61.525) (width 1) (layer F.Cu) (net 1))
 (segment (start 107.5 61.5125) (end 110.9875 61.5125) (width 1) (layer F.Cu) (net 1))
 (segment (start 111 61.525) (end 115 61.525) (width 1) (layer F.Cu) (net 1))
 (segment (start 115 61.525) (end 118.5 61.525) (width 1) (layer F.Cu) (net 1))
 (segment (start 118.5 61.525) (end 122 61.525) (width 1) (layer F.Cu) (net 1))
 (segment (start 122 61.525) (end 126 61.525) (width 1) (layer F.Cu) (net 1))
 (segment (start 126 61.525) (end 129.5 61.525) (width 1) (layer F.Cu) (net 1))
 (segment (start 129.5 61.525) (end 133.5 61.525) (width 1) (layer F.Cu) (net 1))
 (segment (start 133.5 61.525) (end 137 61.525) (width 1) (layer F.Cu) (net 1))
 (segment (start 112.3 78.68) (end 100.18 78.68) (width 1) (layer F.Cu) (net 1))
 (segment (start 100.18 78.68) (end 98.5 77) (width 1) (layer F.Cu) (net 1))
 (segment (start 98.5 77) (end 98.5 63.5) (width 1) (layer F.Cu) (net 1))
 (segment (start 100.4875 61.5125) (end 107.5 61.5125) (width 1) (layer F.Cu) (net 1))
 (segment (start 98.5 63.5) (end 100.4875 61.5125) (width 1) (layer F.Cu) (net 1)))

